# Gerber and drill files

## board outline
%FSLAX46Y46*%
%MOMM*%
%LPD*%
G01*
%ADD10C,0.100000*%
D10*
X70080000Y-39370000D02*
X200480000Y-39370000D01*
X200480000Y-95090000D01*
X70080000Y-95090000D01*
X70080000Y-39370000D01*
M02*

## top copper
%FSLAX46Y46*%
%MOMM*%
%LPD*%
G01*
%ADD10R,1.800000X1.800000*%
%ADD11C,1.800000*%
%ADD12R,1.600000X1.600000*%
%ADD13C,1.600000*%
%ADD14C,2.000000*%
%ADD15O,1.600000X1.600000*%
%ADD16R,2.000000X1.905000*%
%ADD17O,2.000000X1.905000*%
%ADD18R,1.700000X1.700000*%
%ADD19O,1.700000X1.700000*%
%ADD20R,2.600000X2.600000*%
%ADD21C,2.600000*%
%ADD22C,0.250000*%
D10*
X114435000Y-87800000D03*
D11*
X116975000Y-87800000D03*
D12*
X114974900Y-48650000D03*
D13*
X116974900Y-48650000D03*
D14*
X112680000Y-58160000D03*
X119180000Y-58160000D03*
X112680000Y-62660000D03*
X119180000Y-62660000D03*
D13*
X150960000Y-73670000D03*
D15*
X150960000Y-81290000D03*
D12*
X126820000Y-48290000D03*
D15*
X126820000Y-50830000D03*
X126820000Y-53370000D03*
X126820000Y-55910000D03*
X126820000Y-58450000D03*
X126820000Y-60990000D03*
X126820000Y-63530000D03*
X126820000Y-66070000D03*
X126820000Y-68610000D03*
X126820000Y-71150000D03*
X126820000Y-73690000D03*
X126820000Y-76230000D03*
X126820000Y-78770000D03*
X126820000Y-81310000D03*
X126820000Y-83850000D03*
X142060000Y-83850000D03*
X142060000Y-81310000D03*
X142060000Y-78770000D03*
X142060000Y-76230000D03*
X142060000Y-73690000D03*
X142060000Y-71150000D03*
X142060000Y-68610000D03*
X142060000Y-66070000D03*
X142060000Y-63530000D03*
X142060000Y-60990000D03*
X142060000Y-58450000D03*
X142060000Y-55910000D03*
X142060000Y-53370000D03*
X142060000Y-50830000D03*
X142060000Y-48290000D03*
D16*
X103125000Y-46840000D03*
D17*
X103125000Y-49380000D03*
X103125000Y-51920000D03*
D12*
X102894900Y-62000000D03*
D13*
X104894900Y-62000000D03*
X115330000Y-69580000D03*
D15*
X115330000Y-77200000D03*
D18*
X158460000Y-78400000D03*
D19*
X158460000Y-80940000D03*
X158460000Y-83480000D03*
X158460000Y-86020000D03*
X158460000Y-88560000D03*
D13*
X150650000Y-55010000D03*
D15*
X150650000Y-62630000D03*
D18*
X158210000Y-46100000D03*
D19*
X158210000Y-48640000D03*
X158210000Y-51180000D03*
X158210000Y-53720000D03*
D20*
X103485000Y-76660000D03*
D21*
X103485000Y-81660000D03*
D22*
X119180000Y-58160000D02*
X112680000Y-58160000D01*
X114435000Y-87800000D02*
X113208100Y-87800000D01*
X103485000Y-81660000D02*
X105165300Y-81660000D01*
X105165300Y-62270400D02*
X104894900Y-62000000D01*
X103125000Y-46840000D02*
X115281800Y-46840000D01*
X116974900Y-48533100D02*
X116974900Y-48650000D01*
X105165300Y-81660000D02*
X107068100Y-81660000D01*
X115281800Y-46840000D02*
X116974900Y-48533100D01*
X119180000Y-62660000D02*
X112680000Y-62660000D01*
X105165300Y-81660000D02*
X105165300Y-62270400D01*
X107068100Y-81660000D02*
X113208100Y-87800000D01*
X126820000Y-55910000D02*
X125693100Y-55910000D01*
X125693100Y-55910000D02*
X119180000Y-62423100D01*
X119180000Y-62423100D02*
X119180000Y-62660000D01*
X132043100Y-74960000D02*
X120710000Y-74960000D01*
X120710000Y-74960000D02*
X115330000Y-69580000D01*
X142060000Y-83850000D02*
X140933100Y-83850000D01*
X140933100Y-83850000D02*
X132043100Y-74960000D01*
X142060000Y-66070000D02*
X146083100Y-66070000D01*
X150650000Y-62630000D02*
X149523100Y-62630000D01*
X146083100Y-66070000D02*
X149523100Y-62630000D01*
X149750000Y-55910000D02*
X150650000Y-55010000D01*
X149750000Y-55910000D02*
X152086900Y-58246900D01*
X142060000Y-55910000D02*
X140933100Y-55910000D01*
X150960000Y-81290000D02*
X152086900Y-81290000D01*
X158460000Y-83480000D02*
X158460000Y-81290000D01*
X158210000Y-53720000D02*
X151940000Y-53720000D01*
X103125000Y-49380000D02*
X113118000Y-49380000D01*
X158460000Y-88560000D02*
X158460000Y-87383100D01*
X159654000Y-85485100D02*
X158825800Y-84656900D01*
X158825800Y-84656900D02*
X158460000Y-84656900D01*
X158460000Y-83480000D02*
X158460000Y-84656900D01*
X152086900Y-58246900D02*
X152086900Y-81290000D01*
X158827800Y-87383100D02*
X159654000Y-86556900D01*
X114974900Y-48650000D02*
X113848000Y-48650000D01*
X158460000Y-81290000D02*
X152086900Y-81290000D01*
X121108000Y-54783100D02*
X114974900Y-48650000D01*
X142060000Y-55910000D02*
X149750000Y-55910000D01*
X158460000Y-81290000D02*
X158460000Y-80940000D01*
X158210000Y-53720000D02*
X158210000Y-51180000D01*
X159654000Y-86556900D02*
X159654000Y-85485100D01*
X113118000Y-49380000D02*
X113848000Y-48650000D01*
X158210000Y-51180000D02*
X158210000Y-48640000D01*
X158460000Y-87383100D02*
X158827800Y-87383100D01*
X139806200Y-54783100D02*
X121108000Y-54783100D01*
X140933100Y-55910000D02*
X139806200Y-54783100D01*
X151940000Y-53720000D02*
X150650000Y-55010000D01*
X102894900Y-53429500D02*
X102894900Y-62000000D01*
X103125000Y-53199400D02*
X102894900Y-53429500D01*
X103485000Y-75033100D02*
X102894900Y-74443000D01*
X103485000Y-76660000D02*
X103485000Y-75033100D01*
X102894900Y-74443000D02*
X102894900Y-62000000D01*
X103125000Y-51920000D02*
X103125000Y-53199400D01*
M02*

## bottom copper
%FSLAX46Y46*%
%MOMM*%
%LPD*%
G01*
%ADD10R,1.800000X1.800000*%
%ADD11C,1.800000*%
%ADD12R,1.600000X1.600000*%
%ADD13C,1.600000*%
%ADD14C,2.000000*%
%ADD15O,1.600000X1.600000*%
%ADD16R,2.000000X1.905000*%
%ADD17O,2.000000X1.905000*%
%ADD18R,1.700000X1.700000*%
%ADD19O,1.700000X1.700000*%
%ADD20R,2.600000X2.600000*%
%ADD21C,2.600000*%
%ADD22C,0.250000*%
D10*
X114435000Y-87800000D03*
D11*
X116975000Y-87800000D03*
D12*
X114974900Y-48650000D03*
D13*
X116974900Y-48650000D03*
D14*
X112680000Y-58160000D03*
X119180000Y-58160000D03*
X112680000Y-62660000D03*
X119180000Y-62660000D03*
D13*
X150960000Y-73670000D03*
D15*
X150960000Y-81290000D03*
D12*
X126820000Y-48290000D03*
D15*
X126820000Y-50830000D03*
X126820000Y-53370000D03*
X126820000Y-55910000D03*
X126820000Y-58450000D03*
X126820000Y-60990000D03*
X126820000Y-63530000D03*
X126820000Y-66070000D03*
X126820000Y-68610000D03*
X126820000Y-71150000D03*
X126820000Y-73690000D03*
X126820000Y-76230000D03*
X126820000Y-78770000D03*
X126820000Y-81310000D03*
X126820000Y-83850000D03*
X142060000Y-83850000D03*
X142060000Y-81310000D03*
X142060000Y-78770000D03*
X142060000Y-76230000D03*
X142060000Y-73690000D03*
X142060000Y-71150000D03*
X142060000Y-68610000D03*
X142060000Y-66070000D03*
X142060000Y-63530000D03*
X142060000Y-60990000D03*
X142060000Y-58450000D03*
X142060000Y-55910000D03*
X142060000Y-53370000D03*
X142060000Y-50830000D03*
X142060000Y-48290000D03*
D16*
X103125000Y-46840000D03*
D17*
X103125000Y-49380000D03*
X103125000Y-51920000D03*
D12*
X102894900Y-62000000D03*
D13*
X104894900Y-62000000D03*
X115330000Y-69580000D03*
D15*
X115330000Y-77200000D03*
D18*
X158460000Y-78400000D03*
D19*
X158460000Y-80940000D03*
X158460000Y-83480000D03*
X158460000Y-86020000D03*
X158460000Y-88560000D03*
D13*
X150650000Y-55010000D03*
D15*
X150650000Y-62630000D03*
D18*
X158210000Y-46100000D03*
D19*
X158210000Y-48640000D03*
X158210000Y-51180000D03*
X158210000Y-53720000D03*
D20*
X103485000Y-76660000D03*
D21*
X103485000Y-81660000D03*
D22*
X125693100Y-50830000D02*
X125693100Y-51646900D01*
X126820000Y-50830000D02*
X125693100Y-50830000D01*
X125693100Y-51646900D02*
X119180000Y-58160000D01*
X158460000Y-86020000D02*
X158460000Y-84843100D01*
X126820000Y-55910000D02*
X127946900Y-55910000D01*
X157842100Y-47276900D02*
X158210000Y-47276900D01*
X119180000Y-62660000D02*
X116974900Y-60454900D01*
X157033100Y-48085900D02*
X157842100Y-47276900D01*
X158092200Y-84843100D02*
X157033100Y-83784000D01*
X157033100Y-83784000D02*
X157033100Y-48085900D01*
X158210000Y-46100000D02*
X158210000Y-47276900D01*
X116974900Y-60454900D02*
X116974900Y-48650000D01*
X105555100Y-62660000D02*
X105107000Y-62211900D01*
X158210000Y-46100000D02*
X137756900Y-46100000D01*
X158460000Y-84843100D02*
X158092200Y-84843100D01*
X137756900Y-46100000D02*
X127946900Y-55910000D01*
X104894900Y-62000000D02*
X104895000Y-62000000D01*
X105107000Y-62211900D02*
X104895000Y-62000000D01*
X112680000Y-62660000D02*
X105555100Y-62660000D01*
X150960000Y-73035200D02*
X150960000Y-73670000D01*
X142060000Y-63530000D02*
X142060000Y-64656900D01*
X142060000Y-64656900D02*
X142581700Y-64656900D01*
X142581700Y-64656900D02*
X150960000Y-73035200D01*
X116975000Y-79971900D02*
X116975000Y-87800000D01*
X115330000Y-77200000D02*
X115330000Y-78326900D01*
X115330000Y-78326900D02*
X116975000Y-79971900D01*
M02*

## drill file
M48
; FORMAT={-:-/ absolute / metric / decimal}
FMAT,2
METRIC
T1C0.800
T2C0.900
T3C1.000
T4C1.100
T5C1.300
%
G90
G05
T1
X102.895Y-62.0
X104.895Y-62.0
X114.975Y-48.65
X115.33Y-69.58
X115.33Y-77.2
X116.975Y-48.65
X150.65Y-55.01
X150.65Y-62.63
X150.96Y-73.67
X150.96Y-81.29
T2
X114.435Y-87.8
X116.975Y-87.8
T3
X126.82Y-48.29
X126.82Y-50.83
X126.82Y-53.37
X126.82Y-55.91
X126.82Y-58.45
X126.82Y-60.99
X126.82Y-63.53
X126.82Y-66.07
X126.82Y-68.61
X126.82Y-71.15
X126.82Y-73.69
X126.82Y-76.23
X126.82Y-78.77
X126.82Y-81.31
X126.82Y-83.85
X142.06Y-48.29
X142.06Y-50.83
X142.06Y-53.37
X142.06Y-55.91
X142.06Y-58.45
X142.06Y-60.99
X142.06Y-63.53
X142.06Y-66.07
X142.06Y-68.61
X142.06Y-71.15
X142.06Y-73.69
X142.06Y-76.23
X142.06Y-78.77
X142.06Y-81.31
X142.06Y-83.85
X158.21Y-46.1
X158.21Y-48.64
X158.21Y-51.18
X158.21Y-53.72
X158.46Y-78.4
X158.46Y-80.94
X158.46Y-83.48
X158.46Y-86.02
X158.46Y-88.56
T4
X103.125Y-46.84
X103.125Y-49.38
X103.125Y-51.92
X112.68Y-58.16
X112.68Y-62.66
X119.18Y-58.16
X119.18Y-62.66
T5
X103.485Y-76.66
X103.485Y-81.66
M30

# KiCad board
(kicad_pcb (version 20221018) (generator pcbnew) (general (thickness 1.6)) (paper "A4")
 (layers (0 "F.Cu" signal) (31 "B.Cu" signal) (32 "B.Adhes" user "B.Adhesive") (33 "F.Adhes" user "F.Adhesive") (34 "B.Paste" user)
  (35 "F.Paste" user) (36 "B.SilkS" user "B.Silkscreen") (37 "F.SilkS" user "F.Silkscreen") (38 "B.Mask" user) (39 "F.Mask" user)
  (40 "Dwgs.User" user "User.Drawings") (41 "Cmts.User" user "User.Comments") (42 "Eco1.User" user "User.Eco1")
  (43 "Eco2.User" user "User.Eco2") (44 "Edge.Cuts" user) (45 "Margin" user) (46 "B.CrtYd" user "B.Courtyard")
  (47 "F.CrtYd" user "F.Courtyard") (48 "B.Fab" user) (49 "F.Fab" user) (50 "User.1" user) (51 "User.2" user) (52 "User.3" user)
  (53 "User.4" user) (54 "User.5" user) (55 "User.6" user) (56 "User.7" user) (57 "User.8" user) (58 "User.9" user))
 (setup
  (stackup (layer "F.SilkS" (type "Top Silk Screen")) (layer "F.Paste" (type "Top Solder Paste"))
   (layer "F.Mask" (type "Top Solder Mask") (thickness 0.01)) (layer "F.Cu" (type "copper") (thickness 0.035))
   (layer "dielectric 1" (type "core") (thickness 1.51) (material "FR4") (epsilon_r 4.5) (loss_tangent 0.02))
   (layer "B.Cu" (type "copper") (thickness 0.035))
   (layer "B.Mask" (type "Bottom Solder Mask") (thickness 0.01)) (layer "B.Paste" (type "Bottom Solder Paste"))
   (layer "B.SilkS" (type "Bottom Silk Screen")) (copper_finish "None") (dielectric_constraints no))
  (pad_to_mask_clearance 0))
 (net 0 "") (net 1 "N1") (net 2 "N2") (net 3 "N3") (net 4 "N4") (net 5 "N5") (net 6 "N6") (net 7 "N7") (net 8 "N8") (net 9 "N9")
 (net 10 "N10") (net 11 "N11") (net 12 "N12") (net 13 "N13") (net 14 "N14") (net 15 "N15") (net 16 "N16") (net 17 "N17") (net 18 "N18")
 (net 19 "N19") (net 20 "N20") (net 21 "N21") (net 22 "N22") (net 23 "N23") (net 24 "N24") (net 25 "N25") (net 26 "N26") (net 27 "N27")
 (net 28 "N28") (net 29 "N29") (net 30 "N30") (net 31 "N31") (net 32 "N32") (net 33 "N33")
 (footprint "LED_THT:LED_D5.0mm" (layer "F.Cu") (at 114.435 87.8)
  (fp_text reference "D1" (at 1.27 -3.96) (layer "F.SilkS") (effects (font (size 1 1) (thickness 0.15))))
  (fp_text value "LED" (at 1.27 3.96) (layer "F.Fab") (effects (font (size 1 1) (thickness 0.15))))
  (pad "1" thru_hole rect (at 0 0) (size 1.8 1.8) (drill 0.9) (layers "*.Cu" "*.Mask") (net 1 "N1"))
  (pad "2" thru_hole circle (at 2.54 0) (size 1.8 1.8) (drill 0.9) (layers "*.Cu" "*.Mask") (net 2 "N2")))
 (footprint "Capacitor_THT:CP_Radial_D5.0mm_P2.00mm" (layer "F.Cu") (at 114.9749 48.65)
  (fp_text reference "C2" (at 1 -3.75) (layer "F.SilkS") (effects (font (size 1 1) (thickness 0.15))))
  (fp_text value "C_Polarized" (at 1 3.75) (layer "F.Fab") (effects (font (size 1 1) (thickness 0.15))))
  (pad "1" thru_hole rect (at 0 0) (size 1.6 1.6) (drill 0.8) (layers "*.Cu" "*.Mask") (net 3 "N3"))
  (pad "2" thru_hole circle (at 2 0) (size 1.6 1.6) (drill 0.8) (layers "*.Cu" "*.Mask") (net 1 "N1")))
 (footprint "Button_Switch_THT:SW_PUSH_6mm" (layer "F.Cu") (at 112.68 58.16)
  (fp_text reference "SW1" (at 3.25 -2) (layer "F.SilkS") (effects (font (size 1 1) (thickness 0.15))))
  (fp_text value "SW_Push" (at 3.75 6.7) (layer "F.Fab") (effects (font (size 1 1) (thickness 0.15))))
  (pad "1" thru_hole circle (at 0 0 90) (size 2 2) (drill 1.1) (layers "*.Cu" "*.Mask") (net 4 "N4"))
  (pad "1" thru_hole circle (at 6.5 0 90) (size 2 2) (drill 1.1) (layers "*.Cu" "*.Mask") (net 4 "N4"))
  (pad "2" thru_hole circle (at 0 4.5 90) (size 2 2) (drill 1.1) (layers "*.Cu" "*.Mask") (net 1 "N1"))
  (pad "2" thru_hole circle (at 6.5 4.5 90) (size 2 2) (drill 1.1) (layers "*.Cu" "*.Mask") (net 1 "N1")))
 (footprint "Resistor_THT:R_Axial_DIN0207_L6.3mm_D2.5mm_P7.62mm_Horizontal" (layer "F.Cu") (at 150.96 73.67 -90)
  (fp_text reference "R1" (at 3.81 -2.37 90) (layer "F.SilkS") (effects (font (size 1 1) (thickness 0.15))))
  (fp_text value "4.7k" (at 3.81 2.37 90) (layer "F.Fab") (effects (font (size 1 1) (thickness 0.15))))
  (pad "1" thru_hole circle (at 0 0 270) (size 1.6 1.6) (drill 0.8) (layers "*.Cu" "*.Mask") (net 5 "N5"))
  (pad "2" thru_hole oval (at 7.62 0 270) (size 1.6 1.6) (drill 0.8) (layers "*.Cu" "*.Mask") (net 3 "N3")))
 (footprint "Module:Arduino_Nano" (layer "F.Cu") (at 126.82 48.29)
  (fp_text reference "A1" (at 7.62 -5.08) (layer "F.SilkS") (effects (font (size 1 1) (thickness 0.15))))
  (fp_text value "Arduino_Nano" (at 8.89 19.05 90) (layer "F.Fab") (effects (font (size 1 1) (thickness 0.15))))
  (pad "1" thru_hole rect (at 0 0) (size 1.6 1.6) (drill 1) (layers "*.Cu" "*.Mask") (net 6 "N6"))
  (pad "2" thru_hole oval (at 0 2.54) (size 1.6 1.6) (drill 1) (layers "*.Cu" "*.Mask") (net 4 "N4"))
  (pad "3" thru_hole oval (at 0 5.08) (size 1.6 1.6) (drill 1) (layers "*.Cu" "*.Mask") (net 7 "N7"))
  (pad "4" thru_hole oval (at 0 7.62) (size 1.6 1.6) (drill 1) (layers "*.Cu" "*.Mask") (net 1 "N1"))
  (pad "5" thru_hole oval (at 0 10.16) (size 1.6 1.6) (drill 1) (layers "*.Cu" "*.Mask") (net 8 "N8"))
  (pad "6" thru_hole oval (at 0 12.7) (size 1.6 1.6) (drill 1) (layers "*.Cu" "*.Mask") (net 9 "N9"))
  (pad "7" thru_hole oval (at 0 15.24) (size 1.6 1.6) (drill 1) (layers "*.Cu" "*.Mask") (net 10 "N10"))
  (pad "8" thru_hole oval (at 0 17.78) (size 1.6 1.6) (drill 1) (layers "*.Cu" "*.Mask") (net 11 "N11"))
  (pad "9" thru_hole oval (at 0 20.32) (size 1.6 1.6) (drill 1) (layers "*.Cu" "*.Mask") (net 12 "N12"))
  (pad "10" thru_hole oval (at 0 22.86) (size 1.6 1.6) (drill 1) (layers "*.Cu" "*.Mask") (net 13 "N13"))
  (pad "11" thru_hole oval (at 0 25.4) (size 1.6 1.6) (drill 1) (layers "*.Cu" "*.Mask") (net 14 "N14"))
  (pad "12" thru_hole oval (at 0 27.94) (size 1.6 1.6) (drill 1) (layers "*.Cu" "*.Mask") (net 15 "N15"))
  (pad "13" thru_hole oval (at 0 30.48) (size 1.6 1.6) (drill 1) (layers "*.Cu" "*.Mask") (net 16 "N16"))
  (pad "14" thru_hole oval (at 0 33.02) (size 1.6 1.6) (drill 1) (layers "*.Cu" "*.Mask") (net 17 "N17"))
  (pad "15" thru_hole oval (at 0 35.56) (size 1.6 1.6) (drill 1) (layers "*.Cu" "*.Mask") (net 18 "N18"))
  (pad "16" thru_hole oval (at 15.24 35.56) (size 1.6 1.6) (drill 1) (layers "*.Cu" "*.Mask") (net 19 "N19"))
  (pad "17" thru_hole oval (at 15.24 33.02) (size 1.6 1.6) (drill 1) (layers "*.Cu" "*.Mask") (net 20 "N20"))
  (pad "18" thru_hole oval (at 15.24 30.48) (size 1.6 1.6) (drill 1) (layers "*.Cu" "*.Mask") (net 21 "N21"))
  (pad "19" thru_hole oval (at 15.24 27.94) (size 1.6 1.6) (drill 1) (layers "*.Cu" "*.Mask") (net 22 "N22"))
  (pad "20" thru_hole oval (at 15.24 25.4) (size 1.6 1.6) (drill 1) (layers "*.Cu" "*.Mask") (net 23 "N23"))
  (pad "21" thru_hole oval (at 15.24 22.86) (size 1.6 1.6) (drill 1) (layers "*.Cu" "*.Mask") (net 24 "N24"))
  (pad "22" thru_hole oval (at 15.24 20.32) (size 1.6 1.6) (drill 1) (layers "*.Cu" "*.Mask") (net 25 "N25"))
  (pad "23" thru_hole oval (at 15.24 17.78) (size 1.6 1.6) (drill 1) (layers "*.Cu" "*.Mask") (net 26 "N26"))
  (pad "24" thru_hole oval (at 15.24 15.24) (size 1.6 1.6) (drill 1) (layers "*.Cu" "*.Mask") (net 5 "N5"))
  (pad "25" thru_hole oval (at 15.24 12.7) (size 1.6 1.6) (drill 1) (layers "*.Cu" "*.Mask") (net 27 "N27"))
  (pad "26" thru_hole oval (at 15.24 10.16) (size 1.6 1.6) (drill 1) (layers "*.Cu" "*.Mask") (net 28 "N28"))
  (pad "27" thru_hole oval (at 15.24 7.62) (size 1.6 1.6) (drill 1) (layers "*.Cu" "*.Mask") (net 3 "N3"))
  (pad "28" thru_hole oval (at 15.24 5.08) (size 1.6 1.6) (drill 1) (layers "*.Cu" "*.Mask") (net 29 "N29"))
  (pad "29" thru_hole oval (at 15.24 2.54) (size 1.6 1.6) (drill 1) (layers "*.Cu" "*.Mask") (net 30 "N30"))
  (pad "30" thru_hole oval (at 15.24 0) (size 1.6 1.6) (drill 1) (layers "*.Cu" "*.Mask") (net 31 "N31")))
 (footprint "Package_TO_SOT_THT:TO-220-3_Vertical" (layer "F.Cu") (at 103.125 46.84 -90)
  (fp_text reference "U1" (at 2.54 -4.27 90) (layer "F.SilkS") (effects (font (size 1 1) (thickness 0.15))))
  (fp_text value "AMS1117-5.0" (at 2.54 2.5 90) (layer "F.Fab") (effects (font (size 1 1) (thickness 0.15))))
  (pad "1" thru_hole rect (at 0 0 270) (size 1.905 2) (drill 1.1) (layers "*.Cu" "*.Mask") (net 1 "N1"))
  (pad "2" thru_hole oval (at 2.54 0 270) (size 1.905 2) (drill 1.1) (layers "*.Cu" "*.Mask") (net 3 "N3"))
  (pad "3" thru_hole oval (at 5.08 0 270) (size 1.905 2) (drill 1.1) (layers "*.Cu" "*.Mask") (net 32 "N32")))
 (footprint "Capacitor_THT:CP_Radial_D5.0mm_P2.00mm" (layer "F.Cu") (at 102.8949 62)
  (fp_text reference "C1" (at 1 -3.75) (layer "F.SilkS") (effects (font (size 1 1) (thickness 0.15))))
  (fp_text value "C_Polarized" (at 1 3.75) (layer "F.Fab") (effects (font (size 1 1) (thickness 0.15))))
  (pad "1" thru_hole rect (at 0 0) (size 1.6 1.6) (drill 0.8) (layers "*.Cu" "*.Mask") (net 32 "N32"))
  (pad "2" thru_hole circle (at 2 0) (size 1.6 1.6) (drill 0.8) (layers "*.Cu" "*.Mask") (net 1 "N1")))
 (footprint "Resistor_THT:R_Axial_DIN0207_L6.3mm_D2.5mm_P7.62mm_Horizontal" (layer "F.Cu") (at 115.33 69.58 -90)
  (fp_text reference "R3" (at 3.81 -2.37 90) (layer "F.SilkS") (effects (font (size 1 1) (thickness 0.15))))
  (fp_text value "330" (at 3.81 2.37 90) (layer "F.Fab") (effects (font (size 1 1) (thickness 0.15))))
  (pad "1" thru_hole circle (at 0 0 270) (size 1.6 1.6) (drill 0.8) (layers "*.Cu" "*.Mask") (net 19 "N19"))
  (pad "2" thru_hole oval (at 7.62 0 270) (size 1.6 1.6) (drill 0.8) (layers "*.Cu" "*.Mask") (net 2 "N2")))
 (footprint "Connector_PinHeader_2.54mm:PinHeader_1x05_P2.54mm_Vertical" (layer "F.Cu") (at 158.46 78.4)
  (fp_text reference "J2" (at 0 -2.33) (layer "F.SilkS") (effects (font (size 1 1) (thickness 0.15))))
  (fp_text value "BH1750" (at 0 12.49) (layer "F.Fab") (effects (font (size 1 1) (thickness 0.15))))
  (pad "1" thru_hole rect (at 0 0) (size 1.7 1.7) (drill 1) (layers "*.Cu" "*.Mask") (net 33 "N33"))
  (pad "2" thru_hole oval (at 0 2.54) (size 1.7 1.7) (drill 1) (layers "*.Cu" "*.Mask") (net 3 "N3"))
  (pad "3" thru_hole oval (at 0 5.08) (size 1.7 1.7) (drill 1) (layers "*.Cu" "*.Mask") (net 3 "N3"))
  (pad "4" thru_hole oval (at 0 7.62) (size 1.7 1.7) (drill 1) (layers "*.Cu" "*.Mask") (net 1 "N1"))
  (pad "5" thru_hole oval (at 0 10.16) (size 1.7 1.7) (drill 1) (layers "*.Cu" "*.Mask") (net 3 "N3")))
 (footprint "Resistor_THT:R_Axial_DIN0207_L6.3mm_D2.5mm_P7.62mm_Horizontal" (layer "F.Cu") (at 150.65 55.01 -90)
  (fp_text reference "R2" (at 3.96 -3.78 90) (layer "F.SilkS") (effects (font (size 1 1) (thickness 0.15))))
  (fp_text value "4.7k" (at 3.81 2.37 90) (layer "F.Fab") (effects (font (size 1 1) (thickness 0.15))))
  (pad "1" thru_hole circle (at 0 0 270) (size 1.6 1.6) (drill 0.8) (layers "*.Cu" "*.Mask") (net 3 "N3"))
  (pad "2" thru_hole oval (at 7.62 0 270) (size 1.6 1.6) (drill 0.8) (layers "*.Cu" "*.Mask") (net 26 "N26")))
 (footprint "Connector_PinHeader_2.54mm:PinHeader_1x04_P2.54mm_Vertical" (layer "F.Cu") (at 158.21 46.1)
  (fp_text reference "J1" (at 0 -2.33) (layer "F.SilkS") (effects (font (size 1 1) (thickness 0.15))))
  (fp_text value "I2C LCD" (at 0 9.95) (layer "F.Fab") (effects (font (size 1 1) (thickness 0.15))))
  (pad "1" thru_hole rect (at 0 0) (size 1.7 1.7) (drill 1) (layers "*.Cu" "*.Mask") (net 1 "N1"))
  (pad "2" thru_hole oval (at 0 2.54) (size 1.7 1.7) (drill 1) (layers "*.Cu" "*.Mask") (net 3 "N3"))
  (pad "3" thru_hole oval (at 0 5.08) (size 1.7 1.7) (drill 1) (layers "*.Cu" "*.Mask") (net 3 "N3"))
  (pad "4" thru_hole oval (at 0 7.62) (size 1.7 1.7) (drill 1) (layers "*.Cu" "*.Mask") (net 3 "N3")))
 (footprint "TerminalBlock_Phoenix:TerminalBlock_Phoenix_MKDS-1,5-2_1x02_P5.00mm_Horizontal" (layer "F.Cu") (at 103.485 76.66 -90)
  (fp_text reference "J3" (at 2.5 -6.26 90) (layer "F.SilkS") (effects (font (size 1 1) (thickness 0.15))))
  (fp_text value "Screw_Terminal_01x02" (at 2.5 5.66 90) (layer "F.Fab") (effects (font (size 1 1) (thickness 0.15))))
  (pad "1" thru_hole rect (at 0 0 270) (size 2.6 2.6) (drill 1.3) (layers "*.Cu" "*.Mask") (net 32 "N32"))
  (pad "2" thru_hole circle (at 5 0 270) (size 2.6 2.6) (drill 1.3) (layers "*.Cu" "*.Mask") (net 1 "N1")))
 (gr_rect (start 70.08 39.37) (end 200.48 95.09) (stroke (width 0.1) (type default)) (fill none) (layer "Edge.Cuts"))
 (segment (start 119.18 58.16) (end 112.68 58.16) (width 0.25) (layer "F.Cu") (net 4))
 (segment (start 125.6931 50.83) (end 125.6931 51.6469) (width 0.25) (layer "B.Cu") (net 4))
 (segment (start 126.82 50.83) (end 125.6931 50.83) (width 0.25) (layer "B.Cu") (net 4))
 (segment (start 125.6931 51.6469) (end 119.18 58.16) (width 0.25) (layer "B.Cu") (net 4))
 (segment (start 114.435 87.8) (end 113.2081 87.8) (width 0.25) (layer "F.Cu") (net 1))
 (segment (start 103.485 81.66) (end 105.1653 81.66) (width 0.25) (layer "F.Cu") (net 1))
 (segment (start 105.1653 62.2704) (end 104.8949 62) (width 0.25) (layer "F.Cu") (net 1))
 (segment (start 103.125 46.84) (end 115.2818 46.84) (width 0.25) (layer "F.Cu") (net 1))
 (segment (start 116.9749 48.5331) (end 116.9749 48.65) (width 0.25) (layer "F.Cu") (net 1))
 (segment (start 105.1653 81.66) (end 107.0681 81.66) (width 0.25) (layer "F.Cu") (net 1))
 (segment (start 115.2818 46.84) (end 116.9749 48.5331) (width 0.25) (layer "F.Cu") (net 1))
 (segment (start 119.18 62.66) (end 112.68 62.66) (width 0.25) (layer "F.Cu") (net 1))
 (segment (start 105.1653 81.66) (end 105.1653 62.2704) (width 0.25) (layer "F.Cu") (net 1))
 (segment (start 107.0681 81.66) (end 113.2081 87.8) (width 0.25) (layer "F.Cu") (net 1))
 (segment (start 126.82 55.91) (end 125.6931 55.91) (width 0.25) (layer "F.Cu") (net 1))
 (segment (start 125.6931 55.91) (end 119.18 62.4231) (width 0.25) (layer "F.Cu") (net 1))
 (segment (start 119.18 62.4231) (end 119.18 62.66) (width 0.25) (layer "F.Cu") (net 1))
 (segment (start 158.46 86.02) (end 158.46 84.8431) (width 0.25) (layer "B.Cu") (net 1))
 (segment (start 126.82 55.91) (end 127.9469 55.91) (width 0.25) (layer "B.Cu") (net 1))
 (segment (start 157.8421 47.2769) (end 158.21 47.2769) (width 0.25) (layer "B.Cu") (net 1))
 (segment (start 119.18 62.66) (end 116.9749 60.4549) (width 0.25) (layer "B.Cu") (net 1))
 (segment (start 157.0331 48.0859) (end 157.8421 47.2769) (width 0.25) (layer "B.Cu") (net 1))
 (segment (start 158.0922 84.8431) (end 157.0331 83.784) (width 0.25) (layer "B.Cu") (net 1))
 (segment (start 157.0331 83.784) (end 157.0331 48.0859) (width 0.25) (layer "B.Cu") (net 1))
 (segment (start 158.21 46.1) (end 158.21 47.2769) (width 0.25) (layer "B.Cu") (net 1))
 (segment (start 116.9749 60.4549) (end 116.9749 48.65) (width 0.25) (layer "B.Cu") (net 1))
 (segment (start 105.5551 62.66) (end 105.107 62.2119) (width 0.25) (layer "B.Cu") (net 1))
 (segment (start 158.21 46.1) (end 137.7569 46.1) (width 0.25) (layer "B.Cu") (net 1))
 (segment (start 158.46 84.8431) (end 158.0922 84.8431) (width 0.25) (layer "B.Cu") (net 1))
 (segment (start 137.7569 46.1) (end 127.9469 55.91) (width 0.25) (layer "B.Cu") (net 1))
 (segment (start 104.8949 62) (end 104.895 62) (width 0.25) (layer "B.Cu") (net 1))
 (segment (start 105.107 62.2119) (end 104.895 62) (width 0.25) (layer "B.Cu") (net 1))
 (segment (start 112.68 62.66) (end 105.5551 62.66) (width 0.25) (layer "B.Cu") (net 1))
 (segment (start 132.0431 74.96) (end 120.71 74.96) (width 0.25) (layer "F.Cu") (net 19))
 (segment (start 120.71 74.96) (end 115.33 69.58) (width 0.25) (layer "F.Cu") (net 19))
 (segment (start 142.06 83.85) (end 140.9331 83.85) (width 0.25) (layer "F.Cu") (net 19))
 (segment (start 140.9331 83.85) (end 132.0431 74.96) (width 0.25) (layer "F.Cu") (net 19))
 (segment (start 142.06 66.07) (end 146.0831 66.07) (width 0.25) (layer "F.Cu") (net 26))
 (segment (start 150.65 62.63) (end 149.5231 62.63) (width 0.25) (layer "F.Cu") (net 26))
 (segment (start 146.0831 66.07) (end 149.5231 62.63) (width 0.25) (layer "F.Cu") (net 26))
 (segment (start 150.96 73.0352) (end 150.96 73.67) (width 0.25) (layer "B.Cu") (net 5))
 (segment (start 142.06 63.53) (end 142.06 64.6569) (width 0.25) (layer "B.Cu") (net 5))
 (segment (start 142.06 64.6569) (end 142.5817 64.6569) (width 0.25) (layer "B.Cu") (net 5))
 (segment (start 142.5817 64.6569) (end 150.96 73.0352) (width 0.25) (layer "B.Cu") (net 5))
 (segment (start 149.75 55.91) (end 150.65 55.01) (width 0.25) (layer "F.Cu") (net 3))
 (segment (start 149.75 55.91) (end 152.0869 58.2469) (width 0.25) (layer "F.Cu") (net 3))
 (segment (start 142.06 55.91) (end 140.9331 55.91) (width 0.25) (layer "F.Cu") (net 3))
 (segment (start 150.96 81.29) (end 152.0869 81.29) (width 0.25) (layer "F.Cu") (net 3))
 (segment (start 158.46 83.48) (end 158.46 81.29) (width 0.25) (layer "F.Cu") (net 3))
 (segment (start 158.21 53.72) (end 151.94 53.72) (width 0.25) (layer "F.Cu") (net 3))
 (segment (start 103.125 49.38) (end 113.118 49.38) (width 0.25) (layer "F.Cu") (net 3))
 (segment (start 158.46 88.56) (end 158.46 87.3831) (width 0.25) (layer "F.Cu") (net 3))
 (segment (start 159.654 85.4851) (end 158.8258 84.6569) (width 0.25) (layer "F.Cu") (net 3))
 (segment (start 158.8258 84.6569) (end 158.46 84.6569) (width 0.25) (layer "F.Cu") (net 3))
 (segment (start 158.46 83.48) (end 158.46 84.6569) (width 0.25) (layer "F.Cu") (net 3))
 (segment (start 152.0869 58.2469) (end 152.0869 81.29) (width 0.25) (layer "F.Cu") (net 3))
 (segment (start 158.8278 87.3831) (end 159.654 86.5569) (width 0.25) (layer "F.Cu") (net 3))
 (segment (start 114.9749 48.65) (end 113.848 48.65) (width 0.25) (layer "F.Cu") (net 3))
 (segment (start 158.46 81.29) (end 152.0869 81.29) (width 0.25) (layer "F.Cu") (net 3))
 (segment (start 121.108 54.7831) (end 114.9749 48.65) (width 0.25) (layer "F.Cu") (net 3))
 (segment (start 142.06 55.91) (end 149.75 55.91) (width 0.25) (layer "F.Cu") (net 3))
 (segment (start 158.46 81.29) (end 158.46 80.94) (width 0.25) (layer "F.Cu") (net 3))
 (segment (start 158.21 53.72) (end 158.21 51.18) (width 0.25) (layer "F.Cu") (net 3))
 (segment (start 159.654 86.5569) (end 159.654 85.4851) (width 0.25) (layer "F.Cu") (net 3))
 (segment (start 113.118 49.38) (end 113.848 48.65) (width 0.25) (layer "F.Cu") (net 3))
 (segment (start 158.21 51.18) (end 158.21 48.64) (width 0.25) (layer "F.Cu") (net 3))
 (segment (start 158.46 87.3831) (end 158.8278 87.3831) (width 0.25) (layer "F.Cu") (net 3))
 (segment (start 139.8062 54.7831) (end 121.108 54.7831) (width 0.25) (layer "F.Cu") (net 3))
 (segment (start 140.9331 55.91) (end 139.8062 54.7831) (width 0.25) (layer "F.Cu") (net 3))
 (segment (start 151.94 53.72) (end 150.65 55.01) (width 0.25) (layer "F.Cu") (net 3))
 (segment (start 102.8949 53.4295) (end 102.8949 62) (width 0.25) (layer "F.Cu") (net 32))
 (segment (start 103.125 53.1994) (end 102.8949 53.4295) (width 0.25) (layer "F.Cu") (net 32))
 (segment (start 103.485 75.0331) (end 102.8949 74.443) (width 0.25) (layer "F.Cu") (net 32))
 (segment (start 103.485 76.66) (end 103.485 75.0331) (width 0.25) (layer "F.Cu") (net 32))
 (segment (start 102.8949 74.443) (end 102.8949 62) (width 0.25) (layer "F.Cu") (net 32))
 (segment (start 103.125 51.92) (end 103.125 53.1994) (width 0.25) (layer "F.Cu") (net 32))
 (segment (start 116.975 79.9719) (end 116.975 87.8) (width 0.25) (layer "B.Cu") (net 2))
 (segment (start 115.33 77.2) (end 115.33 78.3269) (width 0.25) (layer "B.Cu") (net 2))
 (segment (start 115.33 78.3269) (end 116.975 79.9719) (width 0.25) (layer "B.Cu") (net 2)))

